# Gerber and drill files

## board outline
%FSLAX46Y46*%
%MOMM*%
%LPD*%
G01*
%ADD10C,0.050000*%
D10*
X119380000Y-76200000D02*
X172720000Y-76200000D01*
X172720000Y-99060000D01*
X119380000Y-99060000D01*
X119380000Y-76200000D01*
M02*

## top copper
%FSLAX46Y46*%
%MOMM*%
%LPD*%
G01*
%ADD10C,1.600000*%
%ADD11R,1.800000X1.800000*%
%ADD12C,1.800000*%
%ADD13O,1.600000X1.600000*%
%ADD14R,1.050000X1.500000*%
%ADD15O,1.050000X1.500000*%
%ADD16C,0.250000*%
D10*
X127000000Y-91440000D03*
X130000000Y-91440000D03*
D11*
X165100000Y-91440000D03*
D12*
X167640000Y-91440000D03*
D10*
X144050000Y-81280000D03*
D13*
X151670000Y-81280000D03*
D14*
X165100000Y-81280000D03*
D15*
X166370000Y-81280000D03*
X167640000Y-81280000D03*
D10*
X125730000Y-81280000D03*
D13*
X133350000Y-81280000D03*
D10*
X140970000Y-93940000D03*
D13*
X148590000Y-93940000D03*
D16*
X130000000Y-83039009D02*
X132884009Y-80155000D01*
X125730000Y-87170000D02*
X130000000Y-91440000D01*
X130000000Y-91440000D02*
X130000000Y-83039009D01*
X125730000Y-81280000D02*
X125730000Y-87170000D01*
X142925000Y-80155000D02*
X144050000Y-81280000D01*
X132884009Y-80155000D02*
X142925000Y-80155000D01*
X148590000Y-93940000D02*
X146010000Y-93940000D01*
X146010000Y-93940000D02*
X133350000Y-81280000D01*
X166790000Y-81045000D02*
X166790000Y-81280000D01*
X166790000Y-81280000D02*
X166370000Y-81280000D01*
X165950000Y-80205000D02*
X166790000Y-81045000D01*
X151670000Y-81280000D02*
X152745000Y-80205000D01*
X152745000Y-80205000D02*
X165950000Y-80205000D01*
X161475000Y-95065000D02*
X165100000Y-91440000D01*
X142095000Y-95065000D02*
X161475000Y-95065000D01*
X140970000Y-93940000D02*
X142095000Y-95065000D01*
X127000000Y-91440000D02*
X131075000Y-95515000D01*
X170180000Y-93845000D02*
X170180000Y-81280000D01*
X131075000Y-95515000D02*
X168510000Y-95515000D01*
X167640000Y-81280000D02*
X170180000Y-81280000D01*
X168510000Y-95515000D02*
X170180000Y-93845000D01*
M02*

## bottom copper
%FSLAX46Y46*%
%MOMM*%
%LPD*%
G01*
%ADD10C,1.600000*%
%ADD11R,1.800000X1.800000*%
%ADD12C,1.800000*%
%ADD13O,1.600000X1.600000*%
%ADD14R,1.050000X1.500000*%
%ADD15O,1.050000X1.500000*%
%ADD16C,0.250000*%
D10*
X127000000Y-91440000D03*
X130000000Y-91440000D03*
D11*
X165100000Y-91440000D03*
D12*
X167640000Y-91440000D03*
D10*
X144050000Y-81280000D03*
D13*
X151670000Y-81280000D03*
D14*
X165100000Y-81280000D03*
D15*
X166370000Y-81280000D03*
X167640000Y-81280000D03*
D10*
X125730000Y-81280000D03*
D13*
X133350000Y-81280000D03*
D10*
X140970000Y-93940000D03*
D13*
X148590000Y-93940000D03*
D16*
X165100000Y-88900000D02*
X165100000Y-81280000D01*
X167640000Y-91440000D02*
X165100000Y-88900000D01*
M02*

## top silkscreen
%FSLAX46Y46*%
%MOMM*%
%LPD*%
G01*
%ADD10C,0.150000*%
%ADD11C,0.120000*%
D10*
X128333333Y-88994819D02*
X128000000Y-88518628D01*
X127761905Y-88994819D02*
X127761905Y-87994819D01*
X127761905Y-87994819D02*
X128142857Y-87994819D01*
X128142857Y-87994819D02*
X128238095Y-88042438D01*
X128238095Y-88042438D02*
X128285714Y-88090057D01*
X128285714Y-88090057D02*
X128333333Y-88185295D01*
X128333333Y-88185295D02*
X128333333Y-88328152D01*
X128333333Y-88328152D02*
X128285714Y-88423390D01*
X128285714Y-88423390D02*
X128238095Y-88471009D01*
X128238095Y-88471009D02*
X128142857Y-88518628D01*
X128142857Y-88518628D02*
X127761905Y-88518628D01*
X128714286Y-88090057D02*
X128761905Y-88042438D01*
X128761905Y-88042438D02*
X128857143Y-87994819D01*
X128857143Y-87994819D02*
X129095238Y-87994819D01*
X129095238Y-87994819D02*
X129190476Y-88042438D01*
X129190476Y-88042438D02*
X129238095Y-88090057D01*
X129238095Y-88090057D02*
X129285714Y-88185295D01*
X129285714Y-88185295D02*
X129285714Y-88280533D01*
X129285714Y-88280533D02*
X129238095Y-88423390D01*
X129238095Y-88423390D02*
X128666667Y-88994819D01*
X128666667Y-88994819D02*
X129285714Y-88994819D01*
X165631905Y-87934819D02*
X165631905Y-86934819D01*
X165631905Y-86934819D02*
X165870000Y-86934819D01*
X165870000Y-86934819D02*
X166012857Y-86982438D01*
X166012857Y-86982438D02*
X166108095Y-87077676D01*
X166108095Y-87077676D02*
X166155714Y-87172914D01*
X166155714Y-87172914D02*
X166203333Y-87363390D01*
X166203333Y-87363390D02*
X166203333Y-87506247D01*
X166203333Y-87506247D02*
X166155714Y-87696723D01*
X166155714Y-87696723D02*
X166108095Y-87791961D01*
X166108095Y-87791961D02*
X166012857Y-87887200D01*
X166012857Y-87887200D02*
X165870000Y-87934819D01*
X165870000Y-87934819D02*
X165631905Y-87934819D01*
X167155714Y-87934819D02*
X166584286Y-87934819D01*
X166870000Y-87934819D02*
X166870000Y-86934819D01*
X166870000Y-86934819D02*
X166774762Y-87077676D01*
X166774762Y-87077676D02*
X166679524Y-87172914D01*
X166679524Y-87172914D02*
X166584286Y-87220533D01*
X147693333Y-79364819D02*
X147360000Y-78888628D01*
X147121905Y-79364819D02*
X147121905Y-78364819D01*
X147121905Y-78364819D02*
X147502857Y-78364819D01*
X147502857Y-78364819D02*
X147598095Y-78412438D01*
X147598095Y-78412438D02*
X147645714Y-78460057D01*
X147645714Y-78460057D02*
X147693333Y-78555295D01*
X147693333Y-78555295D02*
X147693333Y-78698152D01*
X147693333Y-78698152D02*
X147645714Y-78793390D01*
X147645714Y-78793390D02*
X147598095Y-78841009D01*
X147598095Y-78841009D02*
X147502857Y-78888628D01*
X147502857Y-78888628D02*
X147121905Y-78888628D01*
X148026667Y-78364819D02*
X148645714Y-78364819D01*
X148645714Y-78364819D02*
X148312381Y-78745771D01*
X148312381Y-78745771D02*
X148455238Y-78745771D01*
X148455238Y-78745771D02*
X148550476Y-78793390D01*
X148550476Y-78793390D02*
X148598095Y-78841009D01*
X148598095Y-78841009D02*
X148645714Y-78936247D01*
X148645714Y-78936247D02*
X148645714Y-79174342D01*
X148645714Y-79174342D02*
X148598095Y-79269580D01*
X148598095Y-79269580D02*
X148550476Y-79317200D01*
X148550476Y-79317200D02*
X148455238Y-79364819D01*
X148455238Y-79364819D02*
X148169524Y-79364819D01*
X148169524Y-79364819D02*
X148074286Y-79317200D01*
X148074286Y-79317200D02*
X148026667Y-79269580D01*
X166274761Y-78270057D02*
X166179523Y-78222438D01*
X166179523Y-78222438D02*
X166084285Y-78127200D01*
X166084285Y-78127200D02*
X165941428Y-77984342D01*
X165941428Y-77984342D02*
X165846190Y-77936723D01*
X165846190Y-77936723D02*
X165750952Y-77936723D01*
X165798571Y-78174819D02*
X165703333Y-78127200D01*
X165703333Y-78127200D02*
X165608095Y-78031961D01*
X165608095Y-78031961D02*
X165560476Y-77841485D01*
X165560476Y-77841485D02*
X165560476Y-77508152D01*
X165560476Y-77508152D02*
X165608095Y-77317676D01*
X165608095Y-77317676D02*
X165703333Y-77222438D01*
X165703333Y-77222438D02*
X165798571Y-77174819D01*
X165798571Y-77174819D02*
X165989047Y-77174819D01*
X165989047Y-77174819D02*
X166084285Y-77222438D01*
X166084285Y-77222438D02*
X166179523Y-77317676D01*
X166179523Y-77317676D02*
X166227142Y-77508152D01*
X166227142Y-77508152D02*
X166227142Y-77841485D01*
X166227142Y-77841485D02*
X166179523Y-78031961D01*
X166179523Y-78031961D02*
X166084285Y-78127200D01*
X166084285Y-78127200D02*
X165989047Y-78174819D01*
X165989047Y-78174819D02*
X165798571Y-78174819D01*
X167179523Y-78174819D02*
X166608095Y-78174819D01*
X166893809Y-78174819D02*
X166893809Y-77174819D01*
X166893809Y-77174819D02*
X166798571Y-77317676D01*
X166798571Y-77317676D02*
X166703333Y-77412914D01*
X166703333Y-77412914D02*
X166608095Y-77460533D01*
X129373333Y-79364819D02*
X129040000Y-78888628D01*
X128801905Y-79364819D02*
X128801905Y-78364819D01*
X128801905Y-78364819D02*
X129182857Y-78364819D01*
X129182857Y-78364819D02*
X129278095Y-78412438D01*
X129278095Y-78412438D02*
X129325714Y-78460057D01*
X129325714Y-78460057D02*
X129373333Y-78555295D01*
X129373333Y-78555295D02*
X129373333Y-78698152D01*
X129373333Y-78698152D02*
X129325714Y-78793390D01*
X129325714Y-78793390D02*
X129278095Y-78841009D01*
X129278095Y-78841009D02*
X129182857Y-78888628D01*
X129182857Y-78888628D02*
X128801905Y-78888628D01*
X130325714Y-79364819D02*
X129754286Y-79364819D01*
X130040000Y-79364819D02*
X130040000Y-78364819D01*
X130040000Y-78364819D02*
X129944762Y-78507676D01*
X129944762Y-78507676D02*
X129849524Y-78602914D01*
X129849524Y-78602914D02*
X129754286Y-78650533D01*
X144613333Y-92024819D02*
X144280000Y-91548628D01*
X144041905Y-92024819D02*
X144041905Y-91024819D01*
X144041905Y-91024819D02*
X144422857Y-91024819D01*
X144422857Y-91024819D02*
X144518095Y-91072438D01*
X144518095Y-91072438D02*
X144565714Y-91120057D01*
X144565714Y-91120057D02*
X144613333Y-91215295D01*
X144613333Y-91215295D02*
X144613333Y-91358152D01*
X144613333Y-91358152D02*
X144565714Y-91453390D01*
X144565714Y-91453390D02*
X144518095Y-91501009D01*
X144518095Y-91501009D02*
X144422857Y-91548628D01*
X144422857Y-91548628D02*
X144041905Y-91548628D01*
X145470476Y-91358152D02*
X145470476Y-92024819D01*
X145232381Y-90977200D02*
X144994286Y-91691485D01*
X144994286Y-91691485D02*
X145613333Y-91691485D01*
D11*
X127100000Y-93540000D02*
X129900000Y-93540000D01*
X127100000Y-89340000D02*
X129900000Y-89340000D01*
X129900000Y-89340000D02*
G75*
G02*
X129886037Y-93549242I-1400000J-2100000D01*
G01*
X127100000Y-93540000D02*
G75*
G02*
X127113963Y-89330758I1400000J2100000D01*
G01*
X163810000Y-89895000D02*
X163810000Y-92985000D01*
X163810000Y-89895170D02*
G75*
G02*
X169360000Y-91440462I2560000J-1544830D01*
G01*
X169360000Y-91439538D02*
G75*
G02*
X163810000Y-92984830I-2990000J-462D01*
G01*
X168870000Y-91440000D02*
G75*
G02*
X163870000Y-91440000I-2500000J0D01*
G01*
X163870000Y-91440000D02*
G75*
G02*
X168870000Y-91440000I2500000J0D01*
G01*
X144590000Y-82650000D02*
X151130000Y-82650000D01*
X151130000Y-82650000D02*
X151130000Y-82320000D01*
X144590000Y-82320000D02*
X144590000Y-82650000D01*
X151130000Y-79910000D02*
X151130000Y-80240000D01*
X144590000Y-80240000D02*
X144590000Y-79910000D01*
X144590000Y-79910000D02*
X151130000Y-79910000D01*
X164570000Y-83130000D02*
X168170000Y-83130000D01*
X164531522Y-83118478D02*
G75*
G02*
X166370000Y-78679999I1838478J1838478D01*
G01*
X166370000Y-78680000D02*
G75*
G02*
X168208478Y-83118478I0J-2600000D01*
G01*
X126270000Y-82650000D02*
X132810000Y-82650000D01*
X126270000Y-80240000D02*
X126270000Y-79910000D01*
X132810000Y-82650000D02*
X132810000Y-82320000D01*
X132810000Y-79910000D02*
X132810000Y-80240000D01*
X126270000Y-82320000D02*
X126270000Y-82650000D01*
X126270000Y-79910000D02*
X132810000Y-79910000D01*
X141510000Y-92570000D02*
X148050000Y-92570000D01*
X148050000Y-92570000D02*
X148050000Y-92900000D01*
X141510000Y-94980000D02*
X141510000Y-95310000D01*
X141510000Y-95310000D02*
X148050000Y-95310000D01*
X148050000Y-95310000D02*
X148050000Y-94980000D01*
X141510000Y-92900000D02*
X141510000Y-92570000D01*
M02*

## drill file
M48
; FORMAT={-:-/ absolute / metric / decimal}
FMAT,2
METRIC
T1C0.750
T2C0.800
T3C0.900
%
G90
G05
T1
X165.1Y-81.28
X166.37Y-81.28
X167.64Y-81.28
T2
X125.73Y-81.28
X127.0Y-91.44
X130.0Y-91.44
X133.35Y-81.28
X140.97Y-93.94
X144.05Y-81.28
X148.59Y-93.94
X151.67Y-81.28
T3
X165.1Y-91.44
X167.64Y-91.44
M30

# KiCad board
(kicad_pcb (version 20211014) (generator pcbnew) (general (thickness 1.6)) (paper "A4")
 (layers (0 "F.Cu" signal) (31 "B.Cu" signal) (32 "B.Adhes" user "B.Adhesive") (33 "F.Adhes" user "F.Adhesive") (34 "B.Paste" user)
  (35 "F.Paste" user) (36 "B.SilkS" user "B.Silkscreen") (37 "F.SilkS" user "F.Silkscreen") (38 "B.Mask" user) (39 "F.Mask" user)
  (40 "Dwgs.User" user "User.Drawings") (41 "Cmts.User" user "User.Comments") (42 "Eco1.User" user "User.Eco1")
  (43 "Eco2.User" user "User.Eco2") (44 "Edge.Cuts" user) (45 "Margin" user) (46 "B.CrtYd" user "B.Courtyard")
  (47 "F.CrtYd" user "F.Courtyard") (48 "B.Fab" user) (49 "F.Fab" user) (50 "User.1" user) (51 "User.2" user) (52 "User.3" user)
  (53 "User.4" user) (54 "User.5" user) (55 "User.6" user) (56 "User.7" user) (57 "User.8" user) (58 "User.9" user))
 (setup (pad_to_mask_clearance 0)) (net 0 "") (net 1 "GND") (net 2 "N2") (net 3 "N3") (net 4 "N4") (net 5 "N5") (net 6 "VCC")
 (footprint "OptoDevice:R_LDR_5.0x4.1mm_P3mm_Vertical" (layer "F.Cu") (at 127 91.44)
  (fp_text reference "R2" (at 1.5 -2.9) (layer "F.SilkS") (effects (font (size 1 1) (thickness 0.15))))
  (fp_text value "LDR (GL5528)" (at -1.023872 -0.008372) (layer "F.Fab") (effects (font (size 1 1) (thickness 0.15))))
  (fp_line (start 0.1 2.1) (end 2.9 2.1) (layer "F.SilkS") (width 0.12))
  (fp_line (start 0.1 -2.1) (end 2.9 -2.1) (layer "F.SilkS") (width 0.12))
  (fp_arc (start 2.9 -2.1) (mid 4.023872 0.008372) (end 2.886037 2.109242) (layer "F.SilkS") (width 0.12))
  (fp_arc (start 0.1 2.1) (mid -1.023872 -0.008372) (end 0.113963 -2.109242) (layer "F.SilkS") (width 0.12))
  (pad "1" thru_hole circle (at 0 0) (size 1.6 1.6) (drill 0.8) (layers *.Cu *.Mask) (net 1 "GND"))
  (pad "2" thru_hole circle (at 3 0) (size 1.6 1.6) (drill 0.8) (layers *.Cu *.Mask) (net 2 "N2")))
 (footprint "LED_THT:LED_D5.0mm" (layer "F.Cu") (at 165.1 91.44)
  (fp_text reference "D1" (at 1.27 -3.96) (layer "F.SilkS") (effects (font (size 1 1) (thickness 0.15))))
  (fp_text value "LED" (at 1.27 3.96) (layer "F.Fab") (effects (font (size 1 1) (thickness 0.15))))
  (fp_line (start -1.29 -1.545) (end -1.29 1.545) (layer "F.SilkS") (width 0.12))
  (fp_arc (start -1.29 -1.54483) (mid 2.072002 -2.880433) (end 4.26 0.000462) (layer "F.SilkS") (width 0.12))
  (fp_arc (start 4.26 -0.000462) (mid 2.072002 2.880433) (end -1.29 1.54483) (layer "F.SilkS") (width 0.12))
  (fp_circle (center 1.27 0) (end 3.77 0) (layer "F.SilkS") (width 0.12) (fill none))
  (pad "1" thru_hole rect (at 0 0) (size 1.8 1.8) (drill 0.9) (layers *.Cu *.Mask) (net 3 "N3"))
  (pad "2" thru_hole circle (at 2.54 0) (size 1.8 1.8) (drill 0.9) (layers *.Cu *.Mask) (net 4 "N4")))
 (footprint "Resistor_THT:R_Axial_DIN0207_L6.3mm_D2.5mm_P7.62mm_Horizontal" (layer "F.Cu") (at 144.05 81.28)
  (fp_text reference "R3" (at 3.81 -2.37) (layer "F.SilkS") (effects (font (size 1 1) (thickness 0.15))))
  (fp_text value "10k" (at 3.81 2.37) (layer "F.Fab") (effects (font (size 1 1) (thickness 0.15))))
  (fp_line (start 0.54 1.37) (end 7.08 1.37) (layer "F.SilkS") (width 0.12))
  (fp_line (start 7.08 1.37) (end 7.08 1.04) (layer "F.SilkS") (width 0.12))
  (fp_line (start 0.54 1.04) (end 0.54 1.37) (layer "F.SilkS") (width 0.12))
  (fp_line (start 7.08 -1.37) (end 7.08 -1.04) (layer "F.SilkS") (width 0.12))
  (fp_line (start 0.54 -1.04) (end 0.54 -1.37) (layer "F.SilkS") (width 0.12))
  (fp_line (start 0.54 -1.37) (end 7.08 -1.37) (layer "F.SilkS") (width 0.12))
  (pad "1" thru_hole circle (at 0 0) (size 1.6 1.6) (drill 0.8) (layers *.Cu *.Mask) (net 2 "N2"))
  (pad "2" thru_hole oval (at 7.62 0) (size 1.6 1.6) (drill 0.8) (layers *.Cu *.Mask) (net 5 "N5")))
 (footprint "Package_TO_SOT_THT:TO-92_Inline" (layer "F.Cu") (at 165.1 81.28)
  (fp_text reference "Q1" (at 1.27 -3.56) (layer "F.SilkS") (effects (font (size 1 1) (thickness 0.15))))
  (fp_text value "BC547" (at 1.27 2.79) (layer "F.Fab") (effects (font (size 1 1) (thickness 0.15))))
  (fp_line (start -0.53 1.85) (end 3.07 1.85) (layer "F.SilkS") (width 0.12))
  (fp_arc (start -0.568478 1.838478) (mid -1.132087 -0.994977) (end 1.27 -2.6) (layer "F.SilkS") (width 0.12))
  (fp_arc (start 1.27 -2.6) (mid 3.672087 -0.994977) (end 3.108478 1.838478) (layer "F.SilkS") (width 0.12))
  (pad "1" thru_hole rect (at 0 0) (size 1.05 1.5) (drill 0.75) (layers *.Cu *.Mask) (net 4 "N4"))
  (pad "2" thru_hole oval (at 1.27 0) (size 1.05 1.5) (drill 0.75) (layers *.Cu *.Mask) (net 5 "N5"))
  (pad "3" thru_hole oval (at 2.54 0) (size 1.05 1.5) (drill 0.75) (layers *.Cu *.Mask) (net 1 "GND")))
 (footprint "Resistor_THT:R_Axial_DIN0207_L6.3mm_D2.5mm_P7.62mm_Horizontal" (layer "F.Cu") (at 125.73 81.28)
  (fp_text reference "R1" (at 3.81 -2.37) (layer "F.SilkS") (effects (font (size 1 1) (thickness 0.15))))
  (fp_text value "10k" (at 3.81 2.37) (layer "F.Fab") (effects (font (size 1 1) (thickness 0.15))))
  (fp_line (start 0.54 1.37) (end 7.08 1.37) (layer "F.SilkS") (width 0.12))
  (fp_line (start 0.54 -1.04) (end 0.54 -1.37) (layer "F.SilkS") (width 0.12))
  (fp_line (start 7.08 1.37) (end 7.08 1.04) (layer "F.SilkS") (width 0.12))
  (fp_line (start 7.08 -1.37) (end 7.08 -1.04) (layer "F.SilkS") (width 0.12))
  (fp_line (start 0.54 1.04) (end 0.54 1.37) (layer "F.SilkS") (width 0.12))
  (fp_line (start 0.54 -1.37) (end 7.08 -1.37) (layer "F.SilkS") (width 0.12))
  (pad "1" thru_hole circle (at 0 0) (size 1.6 1.6) (drill 0.8) (layers *.Cu *.Mask) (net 2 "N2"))
  (pad "2" thru_hole oval (at 7.62 0) (size 1.6 1.6) (drill 0.8) (layers *.Cu *.Mask) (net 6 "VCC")))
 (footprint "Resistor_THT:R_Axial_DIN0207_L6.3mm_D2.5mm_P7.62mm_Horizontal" (layer "F.Cu") (at 140.97 93.94)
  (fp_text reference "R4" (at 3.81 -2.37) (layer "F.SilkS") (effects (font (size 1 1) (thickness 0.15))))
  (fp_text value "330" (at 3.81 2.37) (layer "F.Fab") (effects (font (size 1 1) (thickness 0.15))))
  (fp_line (start 0.54 -1.37) (end 7.08 -1.37) (layer "F.SilkS") (width 0.12))
  (fp_line (start 7.08 -1.37) (end 7.08 -1.04) (layer "F.SilkS") (width 0.12))
  (fp_line (start 0.54 1.04) (end 0.54 1.37) (layer "F.SilkS") (width 0.12))
  (fp_line (start 0.54 1.37) (end 7.08 1.37) (layer "F.SilkS") (width 0.12))
  (fp_line (start 7.08 1.37) (end 7.08 1.04) (layer "F.SilkS") (width 0.12))
  (fp_line (start 0.54 -1.04) (end 0.54 -1.37) (layer "F.SilkS") (width 0.12))
  (pad "1" thru_hole circle (at 0 0) (size 1.6 1.6) (drill 0.8) (layers *.Cu *.Mask) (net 3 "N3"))
  (pad "2" thru_hole oval (at 7.62 0) (size 1.6 1.6) (drill 0.8) (layers *.Cu *.Mask) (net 6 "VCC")))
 (gr_rect (start 172.72 99.06) (end 119.38 76.2) (layer "Edge.Cuts") (width 0.05) (fill none))
 (segment (start 130 83.039009) (end 132.884009 80.155) (width 0.25) (layer "F.Cu") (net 2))
 (segment (start 125.73 87.17) (end 130 91.44) (width 0.25) (layer "F.Cu") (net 2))
 (segment (start 130 91.44) (end 130 83.039009) (width 0.25) (layer "F.Cu") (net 2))
 (segment (start 125.73 81.28) (end 125.73 87.17) (width 0.25) (layer "F.Cu") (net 2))
 (segment (start 142.925 80.155) (end 144.05 81.28) (width 0.25) (layer "F.Cu") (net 2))
 (segment (start 132.884009 80.155) (end 142.925 80.155) (width 0.25) (layer "F.Cu") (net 2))
 (segment (start 148.59 93.94) (end 146.01 93.94) (width 0.25) (layer "F.Cu") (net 6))
 (segment (start 146.01 93.94) (end 133.35 81.28) (width 0.25) (layer "F.Cu") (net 6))
 (segment (start 166.79 81.045) (end 166.79 81.28) (width 0.25) (layer "F.Cu") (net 5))
 (segment (start 166.79 81.28) (end 166.37 81.28) (width 0.25) (layer "F.Cu") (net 5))
 (segment (start 165.95 80.205) (end 166.79 81.045) (width 0.25) (layer "F.Cu") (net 5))
 (segment (start 151.67 81.28) (end 152.745 80.205) (width 0.25) (layer "F.Cu") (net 5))
 (segment (start 152.745 80.205) (end 165.95 80.205) (width 0.25) (layer "F.Cu") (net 5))
 (segment (start 161.475 95.065) (end 165.1 91.44) (width 0.25) (layer "F.Cu") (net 3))
 (segment (start 142.095 95.065) (end 161.475 95.065) (width 0.25) (layer "F.Cu") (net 3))
 (segment (start 140.97 93.94) (end 142.095 95.065) (width 0.25) (layer "F.Cu") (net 3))
 (segment (start 165.1 88.9) (end 165.1 81.28) (width 0.25) (layer "B.Cu") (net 4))
 (segment (start 167.64 91.44) (end 165.1 88.9) (width 0.25) (layer "B.Cu") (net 4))
 (segment (start 127 91.44) (end 131.075 95.515) (width 0.25) (layer "F.Cu") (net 1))
 (segment (start 170.18 93.845) (end 170.18 81.28) (width 0.25) (layer "F.Cu") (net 1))
 (segment (start 131.075 95.515) (end 168.51 95.515) (width 0.25) (layer "F.Cu") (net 1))
 (segment (start 167.64 81.28) (end 170.18 81.28) (width 0.25) (layer "F.Cu") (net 1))
 (segment (start 168.51 95.515) (end 170.18 93.845) (width 0.25) (layer "F.Cu") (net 1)))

